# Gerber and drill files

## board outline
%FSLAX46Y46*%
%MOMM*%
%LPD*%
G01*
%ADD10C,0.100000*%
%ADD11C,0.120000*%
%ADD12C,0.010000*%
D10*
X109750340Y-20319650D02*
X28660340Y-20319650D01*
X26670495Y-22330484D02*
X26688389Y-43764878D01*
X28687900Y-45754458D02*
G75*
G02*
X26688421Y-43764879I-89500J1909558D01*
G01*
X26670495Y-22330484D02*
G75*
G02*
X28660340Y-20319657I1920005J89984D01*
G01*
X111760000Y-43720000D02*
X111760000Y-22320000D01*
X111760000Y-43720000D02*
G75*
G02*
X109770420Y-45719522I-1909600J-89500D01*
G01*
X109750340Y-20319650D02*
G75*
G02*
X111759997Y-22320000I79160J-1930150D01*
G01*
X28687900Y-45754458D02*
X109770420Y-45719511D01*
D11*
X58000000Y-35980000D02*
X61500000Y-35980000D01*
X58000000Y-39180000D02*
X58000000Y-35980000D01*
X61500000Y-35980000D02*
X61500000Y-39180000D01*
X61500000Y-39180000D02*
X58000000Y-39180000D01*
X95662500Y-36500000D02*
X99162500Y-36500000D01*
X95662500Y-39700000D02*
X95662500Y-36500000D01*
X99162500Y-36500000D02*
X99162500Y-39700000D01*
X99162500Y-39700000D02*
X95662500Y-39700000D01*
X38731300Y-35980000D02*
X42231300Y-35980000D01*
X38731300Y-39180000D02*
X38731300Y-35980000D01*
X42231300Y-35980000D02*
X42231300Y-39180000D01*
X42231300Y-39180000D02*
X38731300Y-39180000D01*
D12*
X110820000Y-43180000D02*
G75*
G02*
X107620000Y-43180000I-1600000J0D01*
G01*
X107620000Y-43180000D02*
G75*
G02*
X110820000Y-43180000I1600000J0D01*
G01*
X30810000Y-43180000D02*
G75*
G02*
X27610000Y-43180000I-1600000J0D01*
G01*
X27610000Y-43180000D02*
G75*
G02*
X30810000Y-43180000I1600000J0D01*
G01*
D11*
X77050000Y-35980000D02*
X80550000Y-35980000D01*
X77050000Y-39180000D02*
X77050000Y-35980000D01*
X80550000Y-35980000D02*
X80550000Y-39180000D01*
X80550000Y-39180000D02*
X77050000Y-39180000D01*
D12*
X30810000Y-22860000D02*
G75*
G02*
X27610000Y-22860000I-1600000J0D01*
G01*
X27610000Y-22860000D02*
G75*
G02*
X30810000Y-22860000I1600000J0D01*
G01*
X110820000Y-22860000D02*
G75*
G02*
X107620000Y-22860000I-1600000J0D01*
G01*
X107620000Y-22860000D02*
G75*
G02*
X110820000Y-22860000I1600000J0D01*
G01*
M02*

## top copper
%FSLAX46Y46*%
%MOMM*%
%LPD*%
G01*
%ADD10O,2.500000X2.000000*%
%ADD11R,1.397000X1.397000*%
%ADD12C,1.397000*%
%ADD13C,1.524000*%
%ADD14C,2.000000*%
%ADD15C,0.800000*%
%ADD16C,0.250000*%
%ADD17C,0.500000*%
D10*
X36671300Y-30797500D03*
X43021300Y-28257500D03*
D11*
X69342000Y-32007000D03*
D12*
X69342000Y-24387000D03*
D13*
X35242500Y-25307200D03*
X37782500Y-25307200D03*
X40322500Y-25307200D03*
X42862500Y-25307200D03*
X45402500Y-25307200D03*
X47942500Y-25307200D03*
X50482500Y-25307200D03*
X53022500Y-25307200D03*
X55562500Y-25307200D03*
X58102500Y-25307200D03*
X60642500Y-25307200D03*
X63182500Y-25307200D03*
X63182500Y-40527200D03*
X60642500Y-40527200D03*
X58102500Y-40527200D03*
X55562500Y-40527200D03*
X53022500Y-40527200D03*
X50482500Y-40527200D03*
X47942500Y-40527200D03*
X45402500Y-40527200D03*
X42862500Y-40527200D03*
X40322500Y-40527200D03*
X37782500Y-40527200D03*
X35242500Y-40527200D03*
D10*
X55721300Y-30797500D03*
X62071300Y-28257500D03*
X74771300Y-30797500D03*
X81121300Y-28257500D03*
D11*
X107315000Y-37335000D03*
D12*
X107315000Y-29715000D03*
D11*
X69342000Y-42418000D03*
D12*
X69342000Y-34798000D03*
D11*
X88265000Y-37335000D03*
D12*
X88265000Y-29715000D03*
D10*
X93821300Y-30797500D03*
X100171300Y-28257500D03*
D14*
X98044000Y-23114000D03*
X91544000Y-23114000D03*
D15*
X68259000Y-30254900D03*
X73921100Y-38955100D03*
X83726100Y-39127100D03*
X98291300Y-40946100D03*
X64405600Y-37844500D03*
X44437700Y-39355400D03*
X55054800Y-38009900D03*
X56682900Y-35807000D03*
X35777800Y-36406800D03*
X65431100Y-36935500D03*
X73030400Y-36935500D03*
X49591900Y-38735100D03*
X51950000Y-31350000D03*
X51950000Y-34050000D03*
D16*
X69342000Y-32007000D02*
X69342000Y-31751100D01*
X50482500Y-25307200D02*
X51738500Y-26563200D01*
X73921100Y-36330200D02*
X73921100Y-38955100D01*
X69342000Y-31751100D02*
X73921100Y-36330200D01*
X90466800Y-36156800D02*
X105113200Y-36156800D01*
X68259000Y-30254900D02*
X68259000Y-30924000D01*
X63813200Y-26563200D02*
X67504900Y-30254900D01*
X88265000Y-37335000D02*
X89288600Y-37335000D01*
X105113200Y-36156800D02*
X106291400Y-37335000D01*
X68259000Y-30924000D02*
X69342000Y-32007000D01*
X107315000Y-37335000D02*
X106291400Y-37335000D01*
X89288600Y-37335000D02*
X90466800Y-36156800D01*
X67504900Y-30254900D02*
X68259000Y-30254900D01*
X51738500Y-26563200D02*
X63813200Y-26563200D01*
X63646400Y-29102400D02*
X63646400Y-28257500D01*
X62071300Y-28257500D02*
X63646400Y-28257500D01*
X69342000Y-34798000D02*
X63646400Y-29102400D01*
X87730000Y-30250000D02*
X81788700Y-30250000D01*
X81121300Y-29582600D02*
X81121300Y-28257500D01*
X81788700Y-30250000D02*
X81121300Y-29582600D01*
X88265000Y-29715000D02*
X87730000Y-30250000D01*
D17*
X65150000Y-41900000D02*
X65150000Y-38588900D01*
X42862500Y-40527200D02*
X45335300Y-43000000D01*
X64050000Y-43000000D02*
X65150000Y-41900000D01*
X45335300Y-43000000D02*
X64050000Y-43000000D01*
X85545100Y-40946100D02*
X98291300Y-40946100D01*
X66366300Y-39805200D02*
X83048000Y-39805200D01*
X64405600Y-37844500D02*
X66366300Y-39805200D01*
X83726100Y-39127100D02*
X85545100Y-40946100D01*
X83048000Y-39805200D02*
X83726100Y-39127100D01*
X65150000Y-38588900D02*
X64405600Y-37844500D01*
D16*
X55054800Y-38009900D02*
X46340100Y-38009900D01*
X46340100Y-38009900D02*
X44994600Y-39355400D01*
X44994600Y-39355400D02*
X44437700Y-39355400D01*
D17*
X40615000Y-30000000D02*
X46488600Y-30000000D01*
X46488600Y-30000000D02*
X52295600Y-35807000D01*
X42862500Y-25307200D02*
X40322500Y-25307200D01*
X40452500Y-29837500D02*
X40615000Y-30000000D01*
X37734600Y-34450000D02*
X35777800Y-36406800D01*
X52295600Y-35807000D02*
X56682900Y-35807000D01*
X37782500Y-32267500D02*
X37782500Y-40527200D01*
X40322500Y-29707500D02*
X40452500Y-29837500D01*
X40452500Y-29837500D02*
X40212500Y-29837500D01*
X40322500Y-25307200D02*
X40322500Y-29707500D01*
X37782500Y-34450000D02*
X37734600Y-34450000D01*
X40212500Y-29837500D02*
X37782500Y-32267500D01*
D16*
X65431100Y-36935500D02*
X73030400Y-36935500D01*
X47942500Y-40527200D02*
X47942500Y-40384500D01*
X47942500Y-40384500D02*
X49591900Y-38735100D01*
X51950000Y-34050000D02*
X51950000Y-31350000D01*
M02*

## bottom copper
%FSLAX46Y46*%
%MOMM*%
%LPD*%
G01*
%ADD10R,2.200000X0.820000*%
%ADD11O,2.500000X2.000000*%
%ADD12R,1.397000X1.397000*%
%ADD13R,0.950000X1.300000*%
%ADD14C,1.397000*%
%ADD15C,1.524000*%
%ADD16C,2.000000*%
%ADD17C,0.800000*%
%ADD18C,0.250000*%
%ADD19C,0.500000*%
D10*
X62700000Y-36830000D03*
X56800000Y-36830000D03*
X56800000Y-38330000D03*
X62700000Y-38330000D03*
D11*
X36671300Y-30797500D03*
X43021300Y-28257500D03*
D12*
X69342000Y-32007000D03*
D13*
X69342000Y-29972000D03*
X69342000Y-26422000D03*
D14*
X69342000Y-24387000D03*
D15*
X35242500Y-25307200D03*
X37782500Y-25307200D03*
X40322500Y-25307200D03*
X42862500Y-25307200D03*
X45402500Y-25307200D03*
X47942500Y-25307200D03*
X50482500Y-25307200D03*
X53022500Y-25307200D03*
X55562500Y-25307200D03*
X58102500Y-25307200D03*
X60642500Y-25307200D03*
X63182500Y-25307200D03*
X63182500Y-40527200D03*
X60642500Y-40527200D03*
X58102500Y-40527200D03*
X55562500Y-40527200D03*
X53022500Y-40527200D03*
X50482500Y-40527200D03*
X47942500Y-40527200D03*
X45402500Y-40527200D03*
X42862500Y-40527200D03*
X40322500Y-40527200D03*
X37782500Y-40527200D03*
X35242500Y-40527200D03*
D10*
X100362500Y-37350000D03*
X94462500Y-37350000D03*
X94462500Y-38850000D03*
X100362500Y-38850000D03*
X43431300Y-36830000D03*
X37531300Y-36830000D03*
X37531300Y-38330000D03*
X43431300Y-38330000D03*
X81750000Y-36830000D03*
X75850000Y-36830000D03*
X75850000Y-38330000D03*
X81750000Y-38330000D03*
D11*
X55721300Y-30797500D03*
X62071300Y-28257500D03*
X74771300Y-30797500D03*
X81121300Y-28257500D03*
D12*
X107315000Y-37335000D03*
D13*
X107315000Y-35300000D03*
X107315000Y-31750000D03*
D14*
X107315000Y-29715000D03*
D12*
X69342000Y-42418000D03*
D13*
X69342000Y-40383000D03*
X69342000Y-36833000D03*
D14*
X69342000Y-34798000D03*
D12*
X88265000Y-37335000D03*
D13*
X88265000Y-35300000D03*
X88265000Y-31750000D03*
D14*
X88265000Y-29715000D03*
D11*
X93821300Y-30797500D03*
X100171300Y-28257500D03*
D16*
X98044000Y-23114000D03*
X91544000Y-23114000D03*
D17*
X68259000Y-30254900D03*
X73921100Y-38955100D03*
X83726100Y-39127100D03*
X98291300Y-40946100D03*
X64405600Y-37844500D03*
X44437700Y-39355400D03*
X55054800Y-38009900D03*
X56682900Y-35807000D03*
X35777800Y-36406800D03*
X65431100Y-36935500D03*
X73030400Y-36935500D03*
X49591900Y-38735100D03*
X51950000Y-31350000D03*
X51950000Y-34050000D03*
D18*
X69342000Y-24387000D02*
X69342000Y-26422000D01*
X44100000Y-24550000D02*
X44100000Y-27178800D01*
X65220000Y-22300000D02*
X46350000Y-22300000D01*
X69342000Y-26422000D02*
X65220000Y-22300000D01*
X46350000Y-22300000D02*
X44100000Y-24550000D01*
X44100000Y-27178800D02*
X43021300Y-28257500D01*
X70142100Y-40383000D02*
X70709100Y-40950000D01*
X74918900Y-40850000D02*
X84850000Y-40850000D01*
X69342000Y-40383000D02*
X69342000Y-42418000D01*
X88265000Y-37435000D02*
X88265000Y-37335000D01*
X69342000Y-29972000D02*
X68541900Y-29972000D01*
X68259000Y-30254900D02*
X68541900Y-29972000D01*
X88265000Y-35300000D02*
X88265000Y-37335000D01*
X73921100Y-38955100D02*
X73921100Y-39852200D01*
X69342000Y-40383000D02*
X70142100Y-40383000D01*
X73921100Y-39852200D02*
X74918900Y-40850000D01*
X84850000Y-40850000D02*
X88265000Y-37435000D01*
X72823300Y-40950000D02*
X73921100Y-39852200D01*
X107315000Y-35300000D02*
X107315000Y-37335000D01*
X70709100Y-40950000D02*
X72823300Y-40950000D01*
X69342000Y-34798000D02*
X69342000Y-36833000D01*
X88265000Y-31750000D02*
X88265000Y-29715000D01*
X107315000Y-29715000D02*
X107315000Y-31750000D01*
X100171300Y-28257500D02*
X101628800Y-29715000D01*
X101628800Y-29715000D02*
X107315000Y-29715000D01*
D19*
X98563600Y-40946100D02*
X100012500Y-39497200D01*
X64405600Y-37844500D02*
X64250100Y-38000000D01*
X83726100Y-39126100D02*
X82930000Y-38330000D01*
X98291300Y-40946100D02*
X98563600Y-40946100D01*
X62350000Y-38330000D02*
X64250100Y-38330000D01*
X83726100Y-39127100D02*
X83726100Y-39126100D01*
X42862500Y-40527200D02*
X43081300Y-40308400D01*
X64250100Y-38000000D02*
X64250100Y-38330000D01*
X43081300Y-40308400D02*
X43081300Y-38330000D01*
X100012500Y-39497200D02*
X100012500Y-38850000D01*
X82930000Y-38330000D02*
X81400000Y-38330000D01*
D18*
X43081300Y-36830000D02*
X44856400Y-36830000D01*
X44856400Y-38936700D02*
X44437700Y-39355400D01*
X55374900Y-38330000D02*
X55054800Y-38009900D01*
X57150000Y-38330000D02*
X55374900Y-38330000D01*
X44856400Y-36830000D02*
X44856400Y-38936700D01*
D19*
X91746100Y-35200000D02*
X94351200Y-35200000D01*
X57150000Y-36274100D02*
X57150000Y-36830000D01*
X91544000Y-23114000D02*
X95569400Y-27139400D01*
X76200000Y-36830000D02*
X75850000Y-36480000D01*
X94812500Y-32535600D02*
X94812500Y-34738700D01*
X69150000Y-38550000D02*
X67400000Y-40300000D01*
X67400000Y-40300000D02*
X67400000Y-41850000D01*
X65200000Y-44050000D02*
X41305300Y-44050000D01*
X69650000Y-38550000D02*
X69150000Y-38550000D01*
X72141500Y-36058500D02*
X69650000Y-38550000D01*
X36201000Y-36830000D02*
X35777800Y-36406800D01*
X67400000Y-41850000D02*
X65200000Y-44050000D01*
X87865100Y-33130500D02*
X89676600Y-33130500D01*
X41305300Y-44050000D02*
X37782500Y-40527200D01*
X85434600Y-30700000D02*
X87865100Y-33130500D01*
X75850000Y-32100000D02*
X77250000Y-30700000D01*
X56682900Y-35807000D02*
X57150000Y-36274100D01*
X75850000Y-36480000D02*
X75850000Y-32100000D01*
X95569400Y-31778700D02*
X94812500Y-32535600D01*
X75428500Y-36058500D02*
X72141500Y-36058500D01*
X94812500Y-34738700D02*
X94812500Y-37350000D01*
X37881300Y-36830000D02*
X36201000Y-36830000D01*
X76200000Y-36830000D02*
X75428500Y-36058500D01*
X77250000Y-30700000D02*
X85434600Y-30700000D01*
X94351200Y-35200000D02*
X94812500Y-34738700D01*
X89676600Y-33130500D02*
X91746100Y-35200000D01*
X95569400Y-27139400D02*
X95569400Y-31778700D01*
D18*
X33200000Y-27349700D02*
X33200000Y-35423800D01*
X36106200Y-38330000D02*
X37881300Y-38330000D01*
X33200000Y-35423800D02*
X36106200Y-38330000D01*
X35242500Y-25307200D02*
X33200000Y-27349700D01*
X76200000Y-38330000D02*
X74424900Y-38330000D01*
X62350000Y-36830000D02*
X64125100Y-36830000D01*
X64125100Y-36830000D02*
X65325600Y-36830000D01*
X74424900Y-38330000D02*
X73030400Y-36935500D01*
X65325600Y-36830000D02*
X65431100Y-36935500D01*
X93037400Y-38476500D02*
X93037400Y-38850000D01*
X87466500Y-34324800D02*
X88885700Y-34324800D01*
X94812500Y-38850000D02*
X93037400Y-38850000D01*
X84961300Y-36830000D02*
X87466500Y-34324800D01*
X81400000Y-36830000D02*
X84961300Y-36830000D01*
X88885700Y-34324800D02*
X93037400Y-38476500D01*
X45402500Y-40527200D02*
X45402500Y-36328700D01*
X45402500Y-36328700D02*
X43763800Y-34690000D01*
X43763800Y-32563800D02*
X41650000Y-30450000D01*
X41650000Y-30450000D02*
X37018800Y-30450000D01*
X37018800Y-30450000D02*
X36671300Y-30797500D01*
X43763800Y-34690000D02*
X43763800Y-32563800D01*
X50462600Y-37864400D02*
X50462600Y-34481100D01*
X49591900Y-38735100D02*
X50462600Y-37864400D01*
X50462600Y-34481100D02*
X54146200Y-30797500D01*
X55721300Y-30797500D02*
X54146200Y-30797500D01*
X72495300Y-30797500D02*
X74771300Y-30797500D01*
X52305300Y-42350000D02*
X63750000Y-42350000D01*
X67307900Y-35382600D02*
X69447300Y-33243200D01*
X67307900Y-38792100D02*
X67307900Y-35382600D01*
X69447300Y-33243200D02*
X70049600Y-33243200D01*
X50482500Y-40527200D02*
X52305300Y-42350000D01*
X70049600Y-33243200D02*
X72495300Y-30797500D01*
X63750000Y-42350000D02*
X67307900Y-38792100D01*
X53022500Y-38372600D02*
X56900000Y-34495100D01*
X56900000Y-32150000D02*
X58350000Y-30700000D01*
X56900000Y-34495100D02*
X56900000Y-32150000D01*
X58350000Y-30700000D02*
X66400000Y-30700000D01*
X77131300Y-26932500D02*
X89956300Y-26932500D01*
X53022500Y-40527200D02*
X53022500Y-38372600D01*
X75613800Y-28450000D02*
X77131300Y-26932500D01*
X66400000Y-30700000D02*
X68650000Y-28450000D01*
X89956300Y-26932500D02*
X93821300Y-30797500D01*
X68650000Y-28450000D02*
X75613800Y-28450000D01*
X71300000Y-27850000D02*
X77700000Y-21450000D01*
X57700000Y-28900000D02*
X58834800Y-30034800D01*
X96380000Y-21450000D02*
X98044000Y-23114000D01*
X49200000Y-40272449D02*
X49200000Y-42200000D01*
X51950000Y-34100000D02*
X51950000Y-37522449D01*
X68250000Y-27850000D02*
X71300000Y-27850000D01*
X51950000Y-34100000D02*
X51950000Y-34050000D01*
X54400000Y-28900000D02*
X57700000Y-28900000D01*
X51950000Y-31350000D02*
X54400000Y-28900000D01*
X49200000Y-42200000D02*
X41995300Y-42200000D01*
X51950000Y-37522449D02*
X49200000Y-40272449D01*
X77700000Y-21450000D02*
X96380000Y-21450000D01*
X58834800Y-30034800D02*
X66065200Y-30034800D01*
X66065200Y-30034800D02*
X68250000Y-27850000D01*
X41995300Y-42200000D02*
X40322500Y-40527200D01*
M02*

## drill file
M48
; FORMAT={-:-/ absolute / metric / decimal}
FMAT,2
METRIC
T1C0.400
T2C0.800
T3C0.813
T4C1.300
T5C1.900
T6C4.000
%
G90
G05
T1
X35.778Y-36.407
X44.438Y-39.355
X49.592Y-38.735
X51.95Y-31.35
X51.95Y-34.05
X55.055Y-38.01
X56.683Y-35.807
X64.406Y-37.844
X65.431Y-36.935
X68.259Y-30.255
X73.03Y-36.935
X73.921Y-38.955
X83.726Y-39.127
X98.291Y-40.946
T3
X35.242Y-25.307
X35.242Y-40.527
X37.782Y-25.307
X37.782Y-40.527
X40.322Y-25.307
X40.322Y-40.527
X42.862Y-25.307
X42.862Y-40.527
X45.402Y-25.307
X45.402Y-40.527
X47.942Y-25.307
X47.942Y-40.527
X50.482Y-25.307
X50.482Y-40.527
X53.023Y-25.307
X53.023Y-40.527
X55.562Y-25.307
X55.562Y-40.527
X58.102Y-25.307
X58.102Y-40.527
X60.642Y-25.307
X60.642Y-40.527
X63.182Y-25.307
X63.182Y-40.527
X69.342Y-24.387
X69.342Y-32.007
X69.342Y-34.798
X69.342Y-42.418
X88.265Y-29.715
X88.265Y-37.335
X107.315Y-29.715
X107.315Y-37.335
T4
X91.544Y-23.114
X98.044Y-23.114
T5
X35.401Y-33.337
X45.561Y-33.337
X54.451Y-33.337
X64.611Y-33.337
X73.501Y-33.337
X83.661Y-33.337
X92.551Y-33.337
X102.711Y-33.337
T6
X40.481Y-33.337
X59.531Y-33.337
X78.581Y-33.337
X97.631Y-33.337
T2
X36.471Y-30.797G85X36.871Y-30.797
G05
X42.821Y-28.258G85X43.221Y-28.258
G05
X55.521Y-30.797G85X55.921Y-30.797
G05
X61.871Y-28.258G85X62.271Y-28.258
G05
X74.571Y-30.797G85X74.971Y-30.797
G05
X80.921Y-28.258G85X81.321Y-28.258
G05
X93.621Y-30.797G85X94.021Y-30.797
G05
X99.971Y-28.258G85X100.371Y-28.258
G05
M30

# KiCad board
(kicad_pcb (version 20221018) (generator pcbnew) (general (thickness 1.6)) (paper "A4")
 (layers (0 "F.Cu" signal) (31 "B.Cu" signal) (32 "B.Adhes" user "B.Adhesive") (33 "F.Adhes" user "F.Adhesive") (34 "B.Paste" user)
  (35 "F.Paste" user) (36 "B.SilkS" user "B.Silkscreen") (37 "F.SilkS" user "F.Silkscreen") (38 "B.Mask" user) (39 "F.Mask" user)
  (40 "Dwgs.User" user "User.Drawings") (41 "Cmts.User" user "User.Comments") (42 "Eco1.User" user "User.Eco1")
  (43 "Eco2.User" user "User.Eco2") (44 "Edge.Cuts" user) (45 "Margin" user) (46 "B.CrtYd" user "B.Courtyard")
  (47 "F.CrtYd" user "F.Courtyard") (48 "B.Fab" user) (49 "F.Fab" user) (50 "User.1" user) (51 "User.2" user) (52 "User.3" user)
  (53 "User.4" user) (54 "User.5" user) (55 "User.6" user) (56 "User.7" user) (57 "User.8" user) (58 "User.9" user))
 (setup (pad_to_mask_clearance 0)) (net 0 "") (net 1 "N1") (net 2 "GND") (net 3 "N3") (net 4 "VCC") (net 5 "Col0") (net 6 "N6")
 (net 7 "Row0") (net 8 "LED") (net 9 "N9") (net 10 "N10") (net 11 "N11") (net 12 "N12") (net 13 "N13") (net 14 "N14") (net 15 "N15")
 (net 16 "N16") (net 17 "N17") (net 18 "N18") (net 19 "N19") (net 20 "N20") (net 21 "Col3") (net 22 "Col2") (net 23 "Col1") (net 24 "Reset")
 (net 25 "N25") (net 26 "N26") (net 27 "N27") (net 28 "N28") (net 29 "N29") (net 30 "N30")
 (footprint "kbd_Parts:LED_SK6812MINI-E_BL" (layer "F.Cu") (at 59.75 37.58)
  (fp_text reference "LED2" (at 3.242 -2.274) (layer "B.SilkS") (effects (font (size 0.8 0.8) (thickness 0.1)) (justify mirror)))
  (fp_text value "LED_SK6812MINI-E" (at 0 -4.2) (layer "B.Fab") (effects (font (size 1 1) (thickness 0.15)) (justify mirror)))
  (fp_line (start -1.75 -1.6) (end 1.75 -1.6) (stroke (width 0.12) (type solid)) (layer "Edge.Cuts"))
  (fp_line (start -1.75 1.6) (end -1.75 -1.6) (stroke (width 0.12) (type solid)) (layer "Edge.Cuts"))
  (fp_line (start 1.75 -1.6) (end 1.75 1.6) (stroke (width 0.12) (type solid)) (layer "Edge.Cuts"))
  (fp_line (start 1.75 1.6) (end -1.75 1.6) (stroke (width 0.12) (type solid)) (layer "Edge.Cuts"))
  (pad "1" smd rect (at 2.6 -0.75) (size 2.2 0.82) (drill (offset 0.35 0)) (layers "B.Cu" "B.Paste" "B.Mask") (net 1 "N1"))
  (pad "2" smd rect (at -2.6 -0.75) (size 2.2 0.82) (drill (offset -0.35 0)) (layers "B.Cu" "B.Paste" "B.Mask") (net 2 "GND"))
  (pad "3" smd rect (at -2.6 0.75) (size 2.2 0.82) (drill (offset -0.35 0)) (layers "B.Cu" "B.Paste" "B.Mask") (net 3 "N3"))
  (pad "4" smd rect (at 2.6 0.75) (size 2.2 0.82) (drill (offset 0.35 0)) (layers "B.Cu" "B.Paste" "B.Mask") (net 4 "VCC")))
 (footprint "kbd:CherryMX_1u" (layer "F.Cu") (at 40.4813 33.3375)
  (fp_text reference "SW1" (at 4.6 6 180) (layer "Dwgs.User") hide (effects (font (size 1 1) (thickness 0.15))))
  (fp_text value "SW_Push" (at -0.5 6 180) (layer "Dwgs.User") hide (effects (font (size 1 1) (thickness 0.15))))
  (pad "" np_thru_hole circle (at -5.08 0 90) (size 1.9 1.9) (drill 1.9) (layers "*.Cu" "*.Mask"))
  (pad "" np_thru_hole circle (at 0 0 90) (size 4 4) (drill 4) (layers "*.Cu" "*.Mask"))
  (pad "" np_thru_hole circle (at 5.08 0 90) (size 1.9 1.9) (drill 1.9) (layers "*.Cu" "*.Mask"))
  (pad "1" thru_hole oval (at -3.81 -2.54) (size 2.5 2) (drill oval 1.2 0.8) (layers "*.Cu" "F.SilkS" "B.Mask") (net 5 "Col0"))
  (pad "2" thru_hole oval (at 2.54 -5.08) (size 2.5 2) (drill oval 1.2 0.8) (layers "*.Cu" "F.SilkS" "B.Mask") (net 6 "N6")))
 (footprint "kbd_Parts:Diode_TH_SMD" (layer "F.Cu") (at 69.342 28.197 90)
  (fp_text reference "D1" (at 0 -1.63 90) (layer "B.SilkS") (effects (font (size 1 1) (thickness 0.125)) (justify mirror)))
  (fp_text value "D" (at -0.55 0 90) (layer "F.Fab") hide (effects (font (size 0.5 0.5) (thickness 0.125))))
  (pad "1" thru_hole rect (at -3.81 0 90) (size 1.397 1.397) (drill 0.8128) (layers "*.Cu" "*.Mask" "F.SilkS") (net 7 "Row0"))
  (pad "1" smd rect (at -1.775 0 90) (size 1.3 0.95) (layers "B.Cu" "B.Paste" "B.Mask") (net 7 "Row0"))
  (pad "2" smd rect (at 1.775 0 90) (size 1.3 0.95) (layers "B.Cu" "B.Paste" "B.Mask") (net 6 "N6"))
  (pad "2" thru_hole circle (at 3.81 0 90) (size 1.397 1.397) (drill 0.8128) (layers "*.Cu" "*.Mask" "F.SilkS") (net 6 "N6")))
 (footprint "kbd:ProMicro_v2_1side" (layer "F.Cu") (at 49.7205 32.9636 90)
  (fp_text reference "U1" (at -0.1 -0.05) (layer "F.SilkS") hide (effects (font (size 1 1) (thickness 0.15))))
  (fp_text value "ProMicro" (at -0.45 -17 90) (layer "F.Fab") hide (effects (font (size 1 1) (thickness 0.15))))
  (pad "1" thru_hole circle (at 7.6564 -14.478 90) (size 1.524 1.524) (drill 0.8128) (layers "*.Cu" "F.SilkS" "B.Mask") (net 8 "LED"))
  (pad "2" thru_hole circle (at 7.6564 -11.938 90) (size 1.524 1.524) (drill 0.8128) (layers "*.Cu" "F.SilkS" "B.Mask") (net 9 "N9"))
  (pad "3" thru_hole circle (at 7.6564 -9.398 90) (size 1.524 1.524) (drill 0.8128) (layers "*.Cu" "F.SilkS" "B.Mask") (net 2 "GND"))
  (pad "4" thru_hole circle (at 7.6564 -6.858 90) (size 1.524 1.524) (drill 0.8128) (layers "*.Cu" "F.SilkS" "B.Mask") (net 2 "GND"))
  (pad "5" thru_hole circle (at 7.6564 -4.318 90) (size 1.524 1.524) (drill 0.8128) (layers "*.Cu" "F.SilkS" "B.Mask") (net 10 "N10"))
  (pad "6" thru_hole circle (at 7.6564 -1.778 90) (size 1.524 1.524) (drill 0.8128) (layers "*.Cu" "F.SilkS" "B.Mask") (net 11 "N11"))
  (pad "7" thru_hole circle (at 7.6564 0.762 90) (size 1.524 1.524) (drill 0.8128) (layers "*.Cu" "F.SilkS" "B.Mask") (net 7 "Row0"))
  (pad "8" thru_hole circle (at 7.6564 3.302 90) (size 1.524 1.524) (drill 0.8128) (layers "*.Cu" "F.SilkS" "B.Mask") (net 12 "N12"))
  (pad "9" thru_hole circle (at 7.6564 5.842 90) (size 1.524 1.524) (drill 0.8128) (layers "*.Cu" "F.SilkS" "B.Mask") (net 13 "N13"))
  (pad "10" thru_hole circle (at 7.6564 8.382 90) (size 1.524 1.524) (drill 0.8128) (layers "*.Cu" "F.SilkS" "B.Mask") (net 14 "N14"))
  (pad "11" thru_hole circle (at 7.6564 10.922 90) (size 1.524 1.524) (drill 0.8128) (layers "*.Cu" "F.SilkS" "B.Mask") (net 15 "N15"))
  (pad "12" thru_hole circle (at 7.6564 13.462 90) (size 1.524 1.524) (drill 0.8128) (layers "*.Cu" "F.SilkS" "B.Mask") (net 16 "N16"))
  (pad "13" thru_hole circle (at -7.5636 13.462 90) (size 1.524 1.524) (drill 0.8128) (layers "*.Cu" "F.SilkS" "B.Mask") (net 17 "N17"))
  (pad "14" thru_hole circle (at -7.5636 10.922 90) (size 1.524 1.524) (drill 0.8128) (layers "*.Cu" "F.SilkS" "B.Mask") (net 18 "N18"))
  (pad "15" thru_hole circle (at -7.5636 8.382 90) (size 1.524 1.524) (drill 0.8128) (layers "*.Cu" "F.SilkS" "B.Mask") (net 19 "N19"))
  (pad "16" thru_hole circle (at -7.5636 5.842 90) (size 1.524 1.524) (drill 0.8128) (layers "*.Cu" "F.SilkS" "B.Mask") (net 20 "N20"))
  (pad "17" thru_hole circle (at -7.5636 3.302 90) (size 1.524 1.524) (drill 0.8128) (layers "*.Cu" "F.SilkS" "B.Mask") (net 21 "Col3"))
  (pad "18" thru_hole circle (at -7.5636 0.762 90) (size 1.524 1.524) (drill 0.8128) (layers "*.Cu" "F.SilkS" "B.Mask") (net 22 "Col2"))
  (pad "19" thru_hole circle (at -7.5636 -1.778 90) (size 1.524 1.524) (drill 0.8128) (layers "*.Cu" "F.SilkS" "B.Mask") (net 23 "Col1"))
  (pad "20" thru_hole circle (at -7.5636 -4.318 90) (size 1.524 1.524) (drill 0.8128) (layers "*.Cu" "F.SilkS" "B.Mask") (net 5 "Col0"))
  (pad "21" thru_hole circle (at -7.5636 -6.858 90) (size 1.524 1.524) (drill 0.8128) (layers "*.Cu" "F.SilkS" "B.Mask") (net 4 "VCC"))
  (pad "22" thru_hole circle (at -7.5636 -9.398 90) (size 1.524 1.524) (drill 0.8128) (layers "*.Cu" "F.SilkS" "B.Mask") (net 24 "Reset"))
  (pad "23" thru_hole circle (at -7.5636 -11.938 90) (size 1.524 1.524) (drill 0.8128) (layers "*.Cu" "F.SilkS" "B.Mask") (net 2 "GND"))
  (pad "24" thru_hole circle (at -7.5636 -14.478 90) (size 1.524 1.524) (drill 0.8128) (layers "*.Cu" "F.SilkS" "B.Mask") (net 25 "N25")))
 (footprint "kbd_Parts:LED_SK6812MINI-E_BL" (layer "F.Cu") (at 97.4125 38.1)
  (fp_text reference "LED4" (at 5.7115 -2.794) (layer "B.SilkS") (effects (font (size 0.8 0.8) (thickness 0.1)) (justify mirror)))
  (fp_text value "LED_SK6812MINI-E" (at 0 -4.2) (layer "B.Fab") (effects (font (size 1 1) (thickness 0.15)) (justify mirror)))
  (fp_line (start -1.75 -1.6) (end 1.75 -1.6) (stroke (width 0.12) (type solid)) (layer "Edge.Cuts"))
  (fp_line (start -1.75 1.6) (end -1.75 -1.6) (stroke (width 0.12) (type solid)) (layer "Edge.Cuts"))
  (fp_line (start 1.75 -1.6) (end 1.75 1.6) (stroke (width 0.12) (type solid)) (layer "Edge.Cuts"))
  (fp_line (start 1.75 1.6) (end -1.75 1.6) (stroke (width 0.12) (type solid)) (layer "Edge.Cuts"))
  (pad "1" smd rect (at 2.6 -0.75) (size 2.2 0.82) (drill (offset 0.35 0)) (layers "B.Cu" "B.Paste" "B.Mask") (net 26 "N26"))
  (pad "2" smd rect (at -2.6 -0.75) (size 2.2 0.82) (drill (offset -0.35 0)) (layers "B.Cu" "B.Paste" "B.Mask") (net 2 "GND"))
  (pad "3" smd rect (at -2.6 0.75) (size 2.2 0.82) (drill (offset -0.35 0)) (layers "B.Cu" "B.Paste" "B.Mask") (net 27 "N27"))
  (pad "4" smd rect (at 2.6 0.75) (size 2.2 0.82) (drill (offset 0.35 0)) (layers "B.Cu" "B.Paste" "B.Mask") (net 4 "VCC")))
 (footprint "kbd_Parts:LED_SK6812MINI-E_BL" (layer "F.Cu") (at 40.4813 37.58)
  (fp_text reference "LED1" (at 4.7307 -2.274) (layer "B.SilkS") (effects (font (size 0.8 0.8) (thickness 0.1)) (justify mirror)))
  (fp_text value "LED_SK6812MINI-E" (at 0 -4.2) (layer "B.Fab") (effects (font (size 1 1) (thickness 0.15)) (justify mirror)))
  (fp_line (start -1.75 -1.6) (end 1.75 -1.6) (stroke (width 0.12) (type solid)) (layer "Edge.Cuts"))
  (fp_line (start -1.75 1.6) (end -1.75 -1.6) (stroke (width 0.12) (type solid)) (layer "Edge.Cuts"))
  (fp_line (start 1.75 -1.6) (end 1.75 1.6) (stroke (width 0.12) (type solid)) (layer "Edge.Cuts"))
  (fp_line (start 1.75 1.6) (end -1.75 1.6) (stroke (width 0.12) (type solid)) (layer "Edge.Cuts"))
  (pad "1" smd rect (at 2.6 -0.75) (size 2.2 0.82) (drill (offset 0.35 0)) (layers "B.Cu" "B.Paste" "B.Mask") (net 3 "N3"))
  (pad "2" smd rect (at -2.6 -0.75) (size 2.2 0.82) (drill (offset -0.35 0)) (layers "B.Cu" "B.Paste" "B.Mask") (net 2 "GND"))
  (pad "3" smd rect (at -2.6 0.75) (size 2.2 0.82) (drill (offset -0.35 0)) (layers "B.Cu" "B.Paste" "B.Mask") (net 8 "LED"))
  (pad "4" smd rect (at 2.6 0.75) (size 2.2 0.82) (drill (offset 0.35 0)) (layers "B.Cu" "B.Paste" "B.Mask") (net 4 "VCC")))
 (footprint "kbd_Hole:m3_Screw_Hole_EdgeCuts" (layer "F.Cu") (at 109.22 43.18)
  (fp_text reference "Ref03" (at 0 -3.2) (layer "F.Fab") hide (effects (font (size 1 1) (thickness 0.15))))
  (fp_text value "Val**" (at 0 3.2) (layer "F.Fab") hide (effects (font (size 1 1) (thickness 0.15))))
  (fp_circle (center 0 0) (end 1.6 0) (stroke (width 0.01) (type solid)) (fill none) (layer "Edge.Cuts")))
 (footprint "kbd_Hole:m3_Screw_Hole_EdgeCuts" (layer "F.Cu") (at 29.21 43.18)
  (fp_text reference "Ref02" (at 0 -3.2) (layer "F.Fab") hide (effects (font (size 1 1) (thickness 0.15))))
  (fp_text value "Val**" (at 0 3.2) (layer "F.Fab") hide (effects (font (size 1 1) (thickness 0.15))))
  (fp_circle (center 0 0) (end 1.6 0) (stroke (width 0.01) (type solid)) (fill none) (layer "Edge.Cuts")))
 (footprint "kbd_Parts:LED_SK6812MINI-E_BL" (layer "F.Cu") (at 78.8 37.58)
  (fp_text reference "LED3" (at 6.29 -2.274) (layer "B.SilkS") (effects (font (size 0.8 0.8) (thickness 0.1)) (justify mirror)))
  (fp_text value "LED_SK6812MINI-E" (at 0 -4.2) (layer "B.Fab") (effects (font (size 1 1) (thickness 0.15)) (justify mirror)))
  (fp_line (start -1.75 -1.6) (end 1.75 -1.6) (stroke (width 0.12) (type solid)) (layer "Edge.Cuts"))
  (fp_line (start -1.75 1.6) (end -1.75 -1.6) (stroke (width 0.12) (type solid)) (layer "Edge.Cuts"))
  (fp_line (start 1.75 -1.6) (end 1.75 1.6) (stroke (width 0.12) (type solid)) (layer "Edge.Cuts"))
  (fp_line (start 1.75 1.6) (end -1.75 1.6) (stroke (width 0.12) (type solid)) (layer "Edge.Cuts"))
  (pad "1" smd rect (at 2.6 -0.75) (size 2.2 0.82) (drill (offset 0.35 0)) (layers "B.Cu" "B.Paste" "B.Mask") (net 27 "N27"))
  (pad "2" smd rect (at -2.6 -0.75) (size 2.2 0.82) (drill (offset -0.35 0)) (layers "B.Cu" "B.Paste" "B.Mask") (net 2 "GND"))
  (pad "3" smd rect (at -2.6 0.75) (size 2.2 0.82) (drill (offset -0.35 0)) (layers "B.Cu" "B.Paste" "B.Mask") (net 1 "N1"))
  (pad "4" smd rect (at 2.6 0.75) (size 2.2 0.82) (drill (offset 0.35 0)) (layers "B.Cu" "B.Paste" "B.Mask") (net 4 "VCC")))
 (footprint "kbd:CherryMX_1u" (layer "F.Cu") (at 59.5313 33.3375)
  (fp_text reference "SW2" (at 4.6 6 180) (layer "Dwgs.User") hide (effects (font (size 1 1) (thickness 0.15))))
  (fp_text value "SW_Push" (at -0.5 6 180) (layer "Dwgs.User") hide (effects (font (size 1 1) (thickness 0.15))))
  (pad "" np_thru_hole circle (at -5.08 0 90) (size 1.9 1.9) (drill 1.9) (layers "*.Cu" "*.Mask"))
  (pad "" np_thru_hole circle (at 0 0 90) (size 4 4) (drill 4) (layers "*.Cu" "*.Mask"))
  (pad "" np_thru_hole circle (at 5.08 0 90) (size 1.9 1.9) (drill 1.9) (layers "*.Cu" "*.Mask"))
  (pad "1" thru_hole oval (at -3.81 -2.54) (size 2.5 2) (drill oval 1.2 0.8) (layers "*.Cu" "F.SilkS" "B.Mask") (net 23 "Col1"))
  (pad "2" thru_hole oval (at 2.54 -5.08) (size 2.5 2) (drill oval 1.2 0.8) (layers "*.Cu" "F.SilkS" "B.Mask") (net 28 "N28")))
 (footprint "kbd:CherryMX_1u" (layer "F.Cu") (at 78.5813 33.3375)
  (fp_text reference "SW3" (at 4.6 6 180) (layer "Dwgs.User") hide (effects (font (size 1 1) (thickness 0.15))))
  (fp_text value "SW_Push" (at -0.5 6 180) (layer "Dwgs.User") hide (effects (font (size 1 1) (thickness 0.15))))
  (pad "" np_thru_hole circle (at -5.08 0 90) (size 1.9 1.9) (drill 1.9) (layers "*.Cu" "*.Mask"))
  (pad "" np_thru_hole circle (at 0 0 90) (size 4 4) (drill 4) (layers "*.Cu" "*.Mask"))
  (pad "" np_thru_hole circle (at 5.08 0 90) (size 1.9 1.9) (drill 1.9) (layers "*.Cu" "*.Mask"))
  (pad "1" thru_hole oval (at -3.81 -2.54) (size 2.5 2) (drill oval 1.2 0.8) (layers "*.Cu" "F.SilkS" "B.Mask") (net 22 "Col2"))
  (pad "2" thru_hole oval (at 2.54 -5.08) (size 2.5 2) (drill oval 1.2 0.8) (layers "*.Cu" "F.SilkS" "B.Mask") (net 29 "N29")))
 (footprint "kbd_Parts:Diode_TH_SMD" (layer "F.Cu") (at 107.315 33.525 90)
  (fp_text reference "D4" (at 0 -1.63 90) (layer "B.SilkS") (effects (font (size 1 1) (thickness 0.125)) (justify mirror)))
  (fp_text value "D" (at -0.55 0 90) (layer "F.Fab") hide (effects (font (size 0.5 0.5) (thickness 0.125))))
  (pad "1" thru_hole rect (at -3.81 0 90) (size 1.397 1.397) (drill 0.8128) (layers "*.Cu" "*.Mask" "F.SilkS") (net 7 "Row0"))
  (pad "1" smd rect (at -1.775 0 90) (size 1.3 0.95) (layers "B.Cu" "B.Paste" "B.Mask") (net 7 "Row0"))
  (pad "2" smd rect (at 1.775 0 90) (size 1.3 0.95) (layers "B.Cu" "B.Paste" "B.Mask") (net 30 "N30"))
  (pad "2" thru_hole circle (at 3.81 0 90) (size 1.397 1.397) (drill 0.8128) (layers "*.Cu" "*.Mask" "F.SilkS") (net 30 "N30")))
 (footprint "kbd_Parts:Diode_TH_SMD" (layer "F.Cu") (at 69.342 38.608 90)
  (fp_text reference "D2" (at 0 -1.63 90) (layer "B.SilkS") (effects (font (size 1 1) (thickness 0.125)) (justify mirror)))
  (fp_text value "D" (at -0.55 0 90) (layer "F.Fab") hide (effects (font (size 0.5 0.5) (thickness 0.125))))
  (pad "1" thru_hole rect (at -3.81 0 90) (size 1.397 1.397) (drill 0.8128) (layers "*.Cu" "*.Mask" "F.SilkS") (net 7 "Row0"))
  (pad "1" smd rect (at -1.775 0 90) (size 1.3 0.95) (layers "B.Cu" "B.Paste" "B.Mask") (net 7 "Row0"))
  (pad "2" smd rect (at 1.775 0 90) (size 1.3 0.95) (layers "B.Cu" "B.Paste" "B.Mask") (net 28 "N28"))
  (pad "2" thru_hole circle (at 3.81 0 90) (size 1.397 1.397) (drill 0.8128) (layers "*.Cu" "*.Mask" "F.SilkS") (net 28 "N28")))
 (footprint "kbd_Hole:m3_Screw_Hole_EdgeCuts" (layer "F.Cu") (at 29.21 22.86)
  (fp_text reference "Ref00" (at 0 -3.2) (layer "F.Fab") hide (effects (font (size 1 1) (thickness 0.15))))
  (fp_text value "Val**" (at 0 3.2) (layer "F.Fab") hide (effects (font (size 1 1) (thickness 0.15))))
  (fp_circle (center 0 0) (end 1.6 0) (stroke (width 0.01) (type solid)) (fill none) (layer "Edge.Cuts")))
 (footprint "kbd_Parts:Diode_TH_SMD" (layer "F.Cu") (at 88.265 33.525 90)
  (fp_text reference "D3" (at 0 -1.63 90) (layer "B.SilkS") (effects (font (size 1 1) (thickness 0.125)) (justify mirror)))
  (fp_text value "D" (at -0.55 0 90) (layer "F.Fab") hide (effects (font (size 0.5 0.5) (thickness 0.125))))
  (pad "1" thru_hole rect (at -3.81 0 90) (size 1.397 1.397) (drill 0.8128) (layers "*.Cu" "*.Mask" "F.SilkS") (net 7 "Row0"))
  (pad "1" smd rect (at -1.775 0 90) (size 1.3 0.95) (layers "B.Cu" "B.Paste" "B.Mask") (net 7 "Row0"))
  (pad "2" smd rect (at 1.775 0 90) (size 1.3 0.95) (layers "B.Cu" "B.Paste" "B.Mask") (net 29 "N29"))
  (pad "2" thru_hole circle (at 3.81 0 90) (size 1.397 1.397) (drill 0.8128) (layers "*.Cu" "*.Mask" "F.SilkS") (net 29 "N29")))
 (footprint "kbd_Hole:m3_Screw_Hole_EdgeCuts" (layer "F.Cu") (at 109.22 22.86)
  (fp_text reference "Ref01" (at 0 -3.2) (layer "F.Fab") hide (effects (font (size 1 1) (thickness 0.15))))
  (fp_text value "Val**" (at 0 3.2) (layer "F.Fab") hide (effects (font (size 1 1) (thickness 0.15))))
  (fp_circle (center 0 0) (end 1.6 0) (stroke (width 0.01) (type solid)) (fill none) (layer "Edge.Cuts")))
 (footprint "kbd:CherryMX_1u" (layer "F.Cu") (at 97.6313 33.3375)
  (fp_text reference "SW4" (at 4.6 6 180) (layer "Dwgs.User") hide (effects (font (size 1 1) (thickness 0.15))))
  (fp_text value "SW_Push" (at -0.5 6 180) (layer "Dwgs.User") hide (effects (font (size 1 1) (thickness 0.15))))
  (pad "" np_thru_hole circle (at -5.08 0 90) (size 1.9 1.9) (drill 1.9) (layers "*.Cu" "*.Mask"))
  (pad "" np_thru_hole circle (at 0 0 90) (size 4 4) (drill 4) (layers "*.Cu" "*.Mask"))
  (pad "" np_thru_hole circle (at 5.08 0 90) (size 1.9 1.9) (drill 1.9) (layers "*.Cu" "*.Mask"))
  (pad "1" thru_hole oval (at -3.81 -2.54) (size 2.5 2) (drill oval 1.2 0.8) (layers "*.Cu" "F.SilkS" "B.Mask") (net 21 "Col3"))
  (pad "2" thru_hole oval (at 2.54 -5.08) (size 2.5 2) (drill oval 1.2 0.8) (layers "*.Cu" "F.SilkS" "B.Mask") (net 30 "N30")))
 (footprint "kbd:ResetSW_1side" (layer "B.Cu") (at 94.794 23.114)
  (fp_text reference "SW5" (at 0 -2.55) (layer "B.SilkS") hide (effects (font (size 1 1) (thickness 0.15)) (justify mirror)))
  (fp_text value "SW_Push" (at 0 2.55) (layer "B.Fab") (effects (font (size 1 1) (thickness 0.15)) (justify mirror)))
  (pad "1" thru_hole circle (at 3.25 0) (size 2 2) (drill 1.3) (layers "*.Cu" "F.Mask") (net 24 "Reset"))
  (pad "2" thru_hole circle (at -3.25 0) (size 2 2) (drill 1.3) (layers "*.Cu" "F.Mask") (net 2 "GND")))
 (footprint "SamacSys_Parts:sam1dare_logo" (layer "B.Cu") (at 74.93 24.384 180)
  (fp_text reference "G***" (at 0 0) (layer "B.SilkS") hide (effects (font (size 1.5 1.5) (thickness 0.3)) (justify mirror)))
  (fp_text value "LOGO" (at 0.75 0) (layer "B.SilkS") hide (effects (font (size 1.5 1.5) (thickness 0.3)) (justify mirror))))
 (gr_line (start 109.75034 20.31965) (end 28.66034 20.31965) (stroke (width 0.1) (type default)) (layer "Edge.Cuts"))
 (gr_line (start 26.670495 22.330484) (end 26.688389 43.764878) (stroke (width 0.1) (type default)) (layer "Edge.Cuts"))
 (gr_arc (start 28.6879 45.754458) (mid 27.25 45.2) (end 26.688389 43.764878) (stroke (width 0.1) (type default)) (layer "Edge.Cuts"))
 (gr_arc (start 26.670495 22.330484) (mid 27.224246 20.8885) (end 28.66034 20.31965) (stroke (width 0.1) (type default)) (layer "Edge.Cuts"))
 (gr_line (start 111.76 43.72) (end 111.76 22.32) (stroke (width 0.1) (type default)) (layer "Edge.Cuts"))
 (gr_arc (start 111.76 43.72) (mid 111.205542 45.1579) (end 109.77042 45.719511) (stroke (width 0.1) (type default)) (layer "Edge.Cuts"))
 (gr_arc (start 109.75034 20.31965) (mid 111.192298 20.880663) (end 111.76 22.32) (stroke (width 0.1) (type default)) (layer "Edge.Cuts"))
 (gr_line (start 28.6879 45.754458) (end 109.77042 45.719511) (stroke (width 0.1) (type default)) (layer "Edge.Cuts"))
 (segment (start 69.342 24.387) (end 69.342 26.422) (width 0.25) (layer "B.Cu") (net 6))
 (segment (start 44.1 24.55) (end 44.1 27.1788) (width 0.25) (layer "B.Cu") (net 6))
 (segment (start 65.22 22.3) (end 46.35 22.3) (width 0.25) (layer "B.Cu") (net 6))
 (segment (start 69.342 26.422) (end 65.22 22.3) (width 0.25) (layer "B.Cu") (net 6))
 (segment (start 46.35 22.3) (end 44.1 24.55) (width 0.25) (layer "B.Cu") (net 6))
 (segment (start 44.1 27.1788) (end 43.0213 28.2575) (width 0.25) (layer "B.Cu") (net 6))
 (segment (start 69.342 32.007) (end 69.342 31.7511) (width 0.25) (layer "F.Cu") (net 7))
 (segment (start 50.4825 25.3072) (end 51.7385 26.5632) (width 0.25) (layer "F.Cu") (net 7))
 (segment (start 73.9211 36.3302) (end 73.9211 38.9551) (width 0.25) (layer "F.Cu") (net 7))
 (segment (start 69.342 31.7511) (end 73.9211 36.3302) (width 0.25) (layer "F.Cu") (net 7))
 (segment (start 90.4668 36.1568) (end 105.1132 36.1568) (width 0.25) (layer "F.Cu") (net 7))
 (segment (start 68.259 30.2549) (end 68.259 30.924) (width 0.25) (layer "F.Cu") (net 7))
 (segment (start 63.8132 26.5632) (end 67.5049 30.2549) (width 0.25) (layer "F.Cu") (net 7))
 (segment (start 88.265 37.335) (end 89.2886 37.335) (width 0.25) (layer "F.Cu") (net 7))
 (segment (start 105.1132 36.1568) (end 106.2914 37.335) (width 0.25) (layer "F.Cu") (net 7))
 (segment (start 68.259 30.924) (end 69.342 32.007) (width 0.25) (layer "F.Cu") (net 7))
 (segment (start 107.315 37.335) (end 106.2914 37.335) (width 0.25) (layer "F.Cu") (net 7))
 (segment (start 89.2886 37.335) (end 90.4668 36.1568) (width 0.25) (layer "F.Cu") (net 7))
 (segment (start 67.5049 30.2549) (end 68.259 30.2549) (width 0.25) (layer "F.Cu") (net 7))
 (segment (start 51.7385 26.5632) (end 63.8132 26.5632) (width 0.25) (layer "F.Cu") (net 7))
 (via (at 68.259 30.2549) (size 0.8) (drill 0.4) (layers "F.Cu" "B.Cu") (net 7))
 (via (at 73.9211 38.9551) (size 0.8) (drill 0.4) (layers "F.Cu" "B.Cu") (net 7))
 (segment (start 70.1421 40.383) (end 70.7091 40.95) (width 0.25) (layer "B.Cu") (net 7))
 (segment (start 74.9189 40.85) (end 84.85 40.85) (width 0.25) (layer "B.Cu") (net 7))
 (segment (start 69.342 40.383) (end 69.342 42.418) (width 0.25) (layer "B.Cu") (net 7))
 (segment (start 88.265 37.435) (end 88.265 37.335) (width 0.25) (layer "B.Cu") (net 7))
 (segment (start 69.342 29.972) (end 68.5419 29.972) (width 0.25) (layer "B.Cu") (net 7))
 (segment (start 68.259 30.2549) (end 68.5419 29.972) (width 0.25) (layer "B.Cu") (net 7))
 (segment (start 88.265 35.3) (end 88.265 37.335) (width 0.25) (layer "B.Cu") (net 7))
 (segment (start 73.9211 38.9551) (end 73.9211 39.8522) (width 0.25) (layer "B.Cu") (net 7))
 (segment (start 69.342 40.383) (end 70.1421 40.383) (width 0.25) (layer "B.Cu") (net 7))
 (segment (start 73.9211 39.8522) (end 74.9189 40.85) (width 0.25) (layer "B.Cu") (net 7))
 (segment (start 84.85 40.85) (end 88.265 37.435) (width 0.25) (layer "B.Cu") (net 7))
 (segment (start 72.8233 40.95) (end 73.9211 39.8522) (width 0.25) (layer "B.Cu") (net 7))
 (segment (start 107.315 35.3) (end 107.315 37.335) (width 0.25) (layer "B.Cu") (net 7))
 (segment (start 70.7091 40.95) (end 72.8233 40.95) (width 0.25) (layer "B.Cu") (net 7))
 (segment (start 63.6464 29.1024) (end 63.6464 28.2575) (width 0.25) (layer "F.Cu") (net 28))
 (segment (start 62.0713 28.2575) (end 63.6464 28.2575) (width 0.25) (layer "F.Cu") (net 28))
 (segment (start 69.342 34.798) (end 63.6464 29.1024) (width 0.25) (layer "F.Cu") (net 28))
 (segment (start 69.342 34.798) (end 69.342 36.833) (width 0.25) (layer "B.Cu") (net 28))
 (segment (start 87.73 30.25) (end 81.7887 30.25) (width 0.25) (layer "F.Cu") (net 29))
 (segment (start 81.1213 29.5826) (end 81.1213 28.2575) (width 0.25) (layer "F.Cu") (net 29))
 (segment (start 81.7887 30.25) (end 81.1213 29.5826) (width 0.25) (layer "F.Cu") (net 29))
 (segment (start 88.265 29.715) (end 87.73 30.25) (width 0.25) (layer "F.Cu") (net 29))
 (segment (start 88.265 31.75) (end 88.265 29.715) (width 0.25) (layer "B.Cu") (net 29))
 (segment (start 107.315 29.715) (end 107.315 31.75) (width 0.25) (layer "B.Cu") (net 30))
 (segment (start 100.1713 28.2575) (end 101.6288 29.715) (width 0.25) (layer "B.Cu") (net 30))
 (segment (start 101.6288 29.715) (end 107.315 29.715) (width 0.25) (layer "B.Cu") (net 30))
 (segment (start 65.15 41.9) (end 65.15 38.5889) (width 0.5) (layer "F.Cu") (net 4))
 (segment (start 42.8625 40.5272) (end 45.3353 43) (width 0.5) (layer "F.Cu") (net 4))
 (segment (start 64.05 43) (end 65.15 41.9) (width 0.5) (layer "F.Cu") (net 4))
 (segment (start 45.3353 43) (end 64.05 43) (width 0.5) (layer "F.Cu") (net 4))
 (segment (start 85.5451 40.9461) (end 98.2913 40.9461) (width 0.5) (layer "F.Cu") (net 4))
 (segment (start 66.3663 39.8052) (end 83.048 39.8052) (width 0.5) (layer "F.Cu") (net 4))
 (segment (start 64.4056 37.8445) (end 66.3663 39.8052) (width 0.5) (layer "F.Cu") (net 4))
 (segment (start 83.7261 39.1271) (end 85.5451 40.9461) (width 0.5) (layer "F.Cu") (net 4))
 (segment (start 83.048 39.8052) (end 83.7261 39.1271) (width 0.5) (layer "F.Cu") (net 4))
 (segment (start 65.15 38.5889) (end 64.4056 37.8445) (width 0.5) (layer "F.Cu") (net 4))
 (via (at 83.7261 39.1271) (size 0.8) (drill 0.4) (layers "F.Cu" "B.Cu") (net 4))
 (via (at 98.2913 40.9461) (size 0.8) (drill 0.4) (layers "F.Cu" "B.Cu") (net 4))
 (via (at 64.4056 37.8445) (size 0.8) (drill 0.4) (layers "F.Cu" "B.Cu") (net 4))
 (segment (start 98.5636 40.9461) (end 100.0125 39.4972) (width 0.5) (layer "B.Cu") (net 4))
 (segment (start 64.4056 37.8445) (end 64.2501 38) (width 0.5) (layer "B.Cu") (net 4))
 (segment (start 83.7261 39.1261) (end 82.93 38.33) (width 0.5) (layer "B.Cu") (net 4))
 (segment (start 98.2913 40.9461) (end 98.5636 40.9461) (width 0.5) (layer "B.Cu") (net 4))
 (segment (start 62.35 38.33) (end 64.2501 38.33) (width 0.5) (layer "B.Cu") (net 4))
 (segment (start 83.7261 39.1271) (end 83.7261 39.1261) (width 0.5) (layer "B.Cu") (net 4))
 (segment (start 42.8625 40.5272) (end 43.0813 40.3084) (width 0.5) (layer "B.Cu") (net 4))
 (segment (start 64.2501 38) (end 64.2501 38.33) (width 0.5) (layer "B.Cu") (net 4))
 (segment (start 43.0813 40.3084) (end 43.0813 38.33) (width 0.5) (layer "B.Cu") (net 4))
 (segment (start 100.0125 39.4972) (end 100.0125 38.85) (width 0.5) (layer "B.Cu") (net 4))
 (segment (start 82.93 38.33) (end 81.4 38.33) (width 0.5) (layer "B.Cu") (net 4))
 (segment (start 55.0548 38.0099) (end 46.3401 38.0099) (width 0.25) (layer "F.Cu") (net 3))
 (segment (start 46.3401 38.0099) (end 44.9946 39.3554) (width 0.25) (layer "F.Cu") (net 3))
 (segment (start 44.9946 39.3554) (end 44.4377 39.3554) (width 0.25) (layer "F.Cu") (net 3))
 (via (at 44.4377 39.3554) (size 0.8) (drill 0.4) (layers "F.Cu" "B.Cu") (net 3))
 (via (at 55.0548 38.0099) (size 0.8) (drill 0.4) (layers "F.Cu" "B.Cu") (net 3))
 (segment (start 43.0813 36.83) (end 44.8564 36.83) (width 0.25) (layer "B.Cu") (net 3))
 (segment (start 44.8564 38.9367) (end 44.4377 39.3554) (width 0.25) (layer "B.Cu") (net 3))
 (segment (start 55.3749 38.33) (end 55.0548 38.0099) (width 0.25) (layer "B.Cu") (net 3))
 (segment (start 57.15 38.33) (end 55.3749 38.33) (width 0.25) (layer "B.Cu") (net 3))
 (segment (start 44.8564 36.83) (end 44.8564 38.9367) (width 0.25) (layer "B.Cu") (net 3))
 (segment (start 40.615 30) (end 46.4886 30) (width 0.5) (layer "F.Cu") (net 2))
 (segment (start 46.4886 30) (end 52.2956 35.807) (width 0.5) (layer "F.Cu") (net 2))
 (segment (start 42.8625 25.3072) (end 40.3225 25.3072) (width 0.5) (layer "F.Cu") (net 2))
 (segment (start 40.4525 29.8375) (end 40.615 30) (width 0.5) (layer "F.Cu") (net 2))
 (segment (start 37.7346 34.45) (end 35.7778 36.4068) (width 0.5) (layer "F.Cu") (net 2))
 (segment (start 52.2956 35.807) (end 56.6829 35.807) (width 0.5) (layer "F.Cu") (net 2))
 (segment (start 37.7825 32.2675) (end 37.7825 40.5272) (width 0.5) (layer "F.Cu") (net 2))
 (segment (start 40.3225 29.7075) (end 40.4525 29.8375) (width 0.5) (layer "F.Cu") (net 2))
 (segment (start 40.4525 29.8375) (end 40.2125 29.8375) (width 0.5) (layer "F.Cu") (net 2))
 (segment (start 40.3225 25.3072) (end 40.3225 29.7075) (width 0.5) (layer "F.Cu") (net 2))
 (segment (start 37.7825 34.45) (end 37.7346 34.45) (width 0.5) (layer "F.Cu") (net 2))
 (segment (start 40.2125 29.8375) (end 37.7825 32.2675) (width 0.5) (layer "F.Cu") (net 2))
 (via (at 56.6829 35.807) (size 0.8) (drill 0.4) (layers "F.Cu" "B.Cu") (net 2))
 (via (at 35.7778 36.4068) (size 0.8) (drill 0.4) (layers "F.Cu" "B.Cu") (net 2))
 (segment (start 91.7461 35.2) (end 94.3512 35.2) (width 0.5) (layer "B.Cu") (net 2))
 (segment (start 57.15 36.2741) (end 57.15 36.83) (width 0.5) (layer "B.Cu") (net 2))
 (segment (start 91.544 23.114) (end 95.5694 27.1394) (width 0.5) (layer "B.Cu") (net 2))
 (segment (start 76.2 36.83) (end 75.85 36.48) (width 0.5) (layer "B.Cu") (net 2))
 (segment (start 94.8125 32.5356) (end 94.8125 34.7387) (width 0.5) (layer "B.Cu") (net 2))
 (segment (start 69.15 38.55) (end 67.4 40.3) (width 0.5) (layer "B.Cu") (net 2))
 (segment (start 67.4 40.3) (end 67.4 41.85) (width 0.5) (layer "B.Cu") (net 2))
 (segment (start 65.2 44.05) (end 41.3053 44.05) (width 0.5) (layer "B.Cu") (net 2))
 (segment (start 69.65 38.55) (end 69.15 38.55) (width 0.5) (layer "B.Cu") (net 2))
 (segment (start 72.1415 36.0585) (end 69.65 38.55) (width 0.5) (layer "B.Cu") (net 2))
 (segment (start 36.201 36.83) (end 35.7778 36.4068) (width 0.5) (layer "B.Cu") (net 2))
 (segment (start 67.4 41.85) (end 65.2 44.05) (width 0.5) (layer "B.Cu") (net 2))
 (segment (start 87.8651 33.1305) (end 89.6766 33.1305) (width 0.5) (layer "B.Cu") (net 2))
 (segment (start 41.3053 44.05) (end 37.7825 40.5272) (width 0.5) (layer "B.Cu") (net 2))
 (segment (start 85.4346 30.7) (end 87.8651 33.1305) (width 0.5) (layer "B.Cu") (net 2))
 (segment (start 75.85 32.1) (end 77.25 30.7) (width 0.5) (layer "B.Cu") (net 2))
 (segment (start 56.6829 35.807) (end 57.15 36.2741) (width 0.5) (layer "B.Cu") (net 2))
 (segment (start 75.85 36.48) (end 75.85 32.1) (width 0.5) (layer "B.Cu") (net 2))
 (segment (start 95.5694 31.7787) (end 94.8125 32.5356) (width 0.5) (layer "B.Cu") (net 2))
 (segment (start 75.4285 36.0585) (end 72.1415 36.0585) (width 0.5) (layer "B.Cu") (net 2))
 (segment (start 94.8125 34.7387) (end 94.8125 37.35) (width 0.5) (layer "B.Cu") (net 2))
 (segment (start 37.8813 36.83) (end 36.201 36.83) (width 0.5) (layer "B.Cu") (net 2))
 (segment (start 76.2 36.83) (end 75.4285 36.0585) (width 0.5) (layer "B.Cu") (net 2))
 (segment (start 77.25 30.7) (end 85.4346 30.7) (width 0.5) (layer "B.Cu") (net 2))
 (segment (start 94.3512 35.2) (end 94.8125 34.7387) (width 0.5) (layer "B.Cu") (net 2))
 (segment (start 89.6766 33.1305) (end 91.7461 35.2) (width 0.5) (layer "B.Cu") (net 2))
 (segment (start 95.5694 27.1394) (end 95.5694 31.7787) (width 0.5) (layer "B.Cu") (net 2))
 (segment (start 33.2 27.3497) (end 33.2 35.4238) (width 0.25) (layer "B.Cu") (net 8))
 (segment (start 36.1062 38.33) (end 37.8813 38.33) (width 0.25) (layer "B.Cu") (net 8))
 (segment (start 33.2 35.4238) (end 36.1062 38.33) (width 0.25) (layer "B.Cu") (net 8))
 (segment (start 35.2425 25.3072) (end 33.2 27.3497) (width 0.25) (layer "B.Cu") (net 8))
 (segment (start 65.4311 36.9355) (end 73.0304 36.9355) (width 0.25) (layer "F.Cu") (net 1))
 (via (at 65.4311 36.9355) (size 0.8) (drill 0.4) (layers "F.Cu" "B.Cu") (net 1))
 (via (at 73.0304 36.9355) (size 0.8) (drill 0.4) (layers "F.Cu" "B.Cu") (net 1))
 (segment (start 76.2 38.33) (end 74.4249 38.33) (width 0.25) (layer "B.Cu") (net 1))
 (segment (start 62.35 36.83) (end 64.1251 36.83) (width 0.25) (layer "B.Cu") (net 1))
 (segment (start 64.1251 36.83) (end 65.3256 36.83) (width 0.25) (layer "B.Cu") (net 1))
 (segment (start 74.4249 38.33) (end 73.0304 36.9355) (width 0.25) (layer "B.Cu") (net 1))
 (segment (start 65.3256 36.83) (end 65.4311 36.9355) (width 0.25) (layer "B.Cu") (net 1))
 (segment (start 93.0374 38.4765) (end 93.0374 38.85) (width 0.25) (layer "B.Cu") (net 27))
 (segment (start 87.4665 34.3248) (end 88.8857 34.3248) (width 0.25) (layer "B.Cu") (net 27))
 (segment (start 94.8125 38.85) (end 93.0374 38.85) (width 0.25) (layer "B.Cu") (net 27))
 (segment (start 84.9613 36.83) (end 87.4665 34.3248) (width 0.25) (layer "B.Cu") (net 27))
 (segment (start 81.4 36.83) (end 84.9613 36.83) (width 0.25) (layer "B.Cu") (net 27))
 (segment (start 88.8857 34.3248) (end 93.0374 38.4765) (width 0.25) (layer "B.Cu") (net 27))
 (segment (start 45.4025 40.5272) (end 45.4025 36.3287) (width 0.25) (layer "B.Cu") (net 5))
 (segment (start 45.4025 36.3287) (end 43.7638 34.69) (width 0.25) (layer "B.Cu") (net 5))
 (segment (start 43.7638 32.5638) (end 41.65 30.45) (width 0.25) (layer "B.Cu") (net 5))
 (segment (start 41.65 30.45) (end 37.0188 30.45) (width 0.25) (layer "B.Cu") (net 5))
 (segment (start 37.0188 30.45) (end 36.6713 30.7975) (width 0.25) (layer "B.Cu") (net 5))
 (segment (start 43.7638 34.69) (end 43.7638 32.5638) (width 0.25) (layer "B.Cu") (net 5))
 (segment (start 47.9425 40.5272) (end 47.9425 40.3845) (width 0.25) (layer "F.Cu") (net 23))
 (segment (start 47.9425 40.3845) (end 49.5919 38.7351) (width 0.25) (layer "F.Cu") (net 23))
 (via (at 49.5919 38.7351) (size 0.8) (drill 0.4) (layers "F.Cu" "B.Cu") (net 23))
 (segment (start 50.4626 37.8644) (end 50.4626 34.4811) (width 0.25) (layer "B.Cu") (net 23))
 (segment (start 49.5919 38.7351) (end 50.4626 37.8644) (width 0.25) (layer "B.Cu") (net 23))
 (segment (start 50.4626 34.4811) (end 54.1462 30.7975) (width 0.25) (layer "B.Cu") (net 23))
 (segment (start 55.7213 30.7975) (end 54.1462 30.7975) (width 0.25) (layer "B.Cu") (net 23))
 (segment (start 72.4953 30.7975) (end 74.7713 30.7975) (width 0.25) (layer "B.Cu") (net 22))
 (segment (start 52.3053 42.35) (end 63.75 42.35) (width 0.25) (layer "B.Cu") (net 22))
 (segment (start 67.3079 35.3826) (end 69.4473 33.2432) (width 0.25) (layer "B.Cu") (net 22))
 (segment (start 67.3079 38.7921) (end 67.3079 35.3826) (width 0.25) (layer "B.Cu") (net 22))
 (segment (start 69.4473 33.2432) (end 70.0496 33.2432) (width 0.25) (layer "B.Cu") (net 22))
 (segment (start 50.4825 40.5272) (end 52.3053 42.35) (width 0.25) (layer "B.Cu") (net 22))
 (segment (start 70.0496 33.2432) (end 72.4953 30.7975) (width 0.25) (layer "B.Cu") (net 22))
 (segment (start 63.75 42.35) (end 67.3079 38.7921) (width 0.25) (layer "B.Cu") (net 22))
 (segment (start 53.0225 38.3726) (end 56.9 34.4951) (width 0.25) (layer "B.Cu") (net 21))
 (segment (start 56.9 32.15) (end 58.35 30.7) (width 0.25) (layer "B.Cu") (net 21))
 (segment (start 56.9 34.4951) (end 56.9 32.15) (width 0.25) (layer "B.Cu") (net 21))
 (segment (start 58.35 30.7) (end 66.4 30.7) (width 0.25) (layer "B.Cu") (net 21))
 (segment (start 77.1313 26.9325) (end 89.9563 26.9325) (width 0.25) (layer "B.Cu") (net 21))
 (segment (start 53.0225 40.5272) (end 53.0225 38.3726) (width 0.25) (layer "B.Cu") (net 21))
 (segment (start 75.6138 28.45) (end 77.1313 26.9325) (width 0.25) (layer "B.Cu") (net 21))
 (segment (start 66.4 30.7) (end 68.65 28.45) (width 0.25) (layer "B.Cu") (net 21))
 (segment (start 89.9563 26.9325) (end 93.8213 30.7975) (width 0.25) (layer "B.Cu") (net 21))
 (segment (start 68.65 28.45) (end 75.6138 28.45) (width 0.25) (layer "B.Cu") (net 21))
 (segment (start 51.95 34.05) (end 51.95 31.35) (width 0.25) (layer "F.Cu") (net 24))
 (via (at 51.95 31.35) (size 0.8) (drill 0.4) (layers "F.Cu" "B.Cu") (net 24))
 (via (at 51.95 34.05) (size 0.8) (drill 0.4) (layers "F.Cu" "B.Cu") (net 24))
 (segment (start 71.3 27.85) (end 77.7 21.45) (width 0.25) (layer "B.Cu") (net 24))
 (segment (start 57.7 28.9) (end 58.8348 30.0348) (width 0.25) (layer "B.Cu") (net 24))
 (segment (start 96.38 21.45) (end 98.044 23.114) (width 0.25) (layer "B.Cu") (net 24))
 (segment (start 49.2 40.272449) (end 49.2 42.2) (width 0.25) (layer "B.Cu") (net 24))
 (segment (start 51.95 34.1) (end 51.95 37.522449) (width 0.25) (layer "B.Cu") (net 24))
 (segment (start 68.25 27.85) (end 71.3 27.85) (width 0.25) (layer "B.Cu") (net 24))
 (segment (start 51.95 34.1) (end 51.95 34.05) (width 0.25) (layer "B.Cu") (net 24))
 (segment (start 54.4 28.9) (end 57.7 28.9) (width 0.25) (layer "B.Cu") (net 24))
 (segment (start 51.95 31.35) (end 54.4 28.9) (width 0.25) (layer "B.Cu") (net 24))
 (segment (start 49.2 42.2) (end 41.9953 42.2) (width 0.25) (layer "B.Cu") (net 24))
 (segment (start 51.95 37.522449) (end 49.2 40.272449) (width 0.25) (layer "B.Cu") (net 24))
 (segment (start 77.7 21.45) (end 96.38 21.45) (width 0.25) (layer "B.Cu") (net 24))
 (segment (start 58.8348 30.0348) (end 66.0652 30.0348) (width 0.25) (layer "B.Cu") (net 24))
 (segment (start 66.0652 30.0348) (end 68.25 27.85) (width 0.25) (layer "B.Cu") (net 24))
 (segment (start 41.9953 42.2) (end 40.3225 40.5272) (width 0.25) (layer "B.Cu") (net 24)))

